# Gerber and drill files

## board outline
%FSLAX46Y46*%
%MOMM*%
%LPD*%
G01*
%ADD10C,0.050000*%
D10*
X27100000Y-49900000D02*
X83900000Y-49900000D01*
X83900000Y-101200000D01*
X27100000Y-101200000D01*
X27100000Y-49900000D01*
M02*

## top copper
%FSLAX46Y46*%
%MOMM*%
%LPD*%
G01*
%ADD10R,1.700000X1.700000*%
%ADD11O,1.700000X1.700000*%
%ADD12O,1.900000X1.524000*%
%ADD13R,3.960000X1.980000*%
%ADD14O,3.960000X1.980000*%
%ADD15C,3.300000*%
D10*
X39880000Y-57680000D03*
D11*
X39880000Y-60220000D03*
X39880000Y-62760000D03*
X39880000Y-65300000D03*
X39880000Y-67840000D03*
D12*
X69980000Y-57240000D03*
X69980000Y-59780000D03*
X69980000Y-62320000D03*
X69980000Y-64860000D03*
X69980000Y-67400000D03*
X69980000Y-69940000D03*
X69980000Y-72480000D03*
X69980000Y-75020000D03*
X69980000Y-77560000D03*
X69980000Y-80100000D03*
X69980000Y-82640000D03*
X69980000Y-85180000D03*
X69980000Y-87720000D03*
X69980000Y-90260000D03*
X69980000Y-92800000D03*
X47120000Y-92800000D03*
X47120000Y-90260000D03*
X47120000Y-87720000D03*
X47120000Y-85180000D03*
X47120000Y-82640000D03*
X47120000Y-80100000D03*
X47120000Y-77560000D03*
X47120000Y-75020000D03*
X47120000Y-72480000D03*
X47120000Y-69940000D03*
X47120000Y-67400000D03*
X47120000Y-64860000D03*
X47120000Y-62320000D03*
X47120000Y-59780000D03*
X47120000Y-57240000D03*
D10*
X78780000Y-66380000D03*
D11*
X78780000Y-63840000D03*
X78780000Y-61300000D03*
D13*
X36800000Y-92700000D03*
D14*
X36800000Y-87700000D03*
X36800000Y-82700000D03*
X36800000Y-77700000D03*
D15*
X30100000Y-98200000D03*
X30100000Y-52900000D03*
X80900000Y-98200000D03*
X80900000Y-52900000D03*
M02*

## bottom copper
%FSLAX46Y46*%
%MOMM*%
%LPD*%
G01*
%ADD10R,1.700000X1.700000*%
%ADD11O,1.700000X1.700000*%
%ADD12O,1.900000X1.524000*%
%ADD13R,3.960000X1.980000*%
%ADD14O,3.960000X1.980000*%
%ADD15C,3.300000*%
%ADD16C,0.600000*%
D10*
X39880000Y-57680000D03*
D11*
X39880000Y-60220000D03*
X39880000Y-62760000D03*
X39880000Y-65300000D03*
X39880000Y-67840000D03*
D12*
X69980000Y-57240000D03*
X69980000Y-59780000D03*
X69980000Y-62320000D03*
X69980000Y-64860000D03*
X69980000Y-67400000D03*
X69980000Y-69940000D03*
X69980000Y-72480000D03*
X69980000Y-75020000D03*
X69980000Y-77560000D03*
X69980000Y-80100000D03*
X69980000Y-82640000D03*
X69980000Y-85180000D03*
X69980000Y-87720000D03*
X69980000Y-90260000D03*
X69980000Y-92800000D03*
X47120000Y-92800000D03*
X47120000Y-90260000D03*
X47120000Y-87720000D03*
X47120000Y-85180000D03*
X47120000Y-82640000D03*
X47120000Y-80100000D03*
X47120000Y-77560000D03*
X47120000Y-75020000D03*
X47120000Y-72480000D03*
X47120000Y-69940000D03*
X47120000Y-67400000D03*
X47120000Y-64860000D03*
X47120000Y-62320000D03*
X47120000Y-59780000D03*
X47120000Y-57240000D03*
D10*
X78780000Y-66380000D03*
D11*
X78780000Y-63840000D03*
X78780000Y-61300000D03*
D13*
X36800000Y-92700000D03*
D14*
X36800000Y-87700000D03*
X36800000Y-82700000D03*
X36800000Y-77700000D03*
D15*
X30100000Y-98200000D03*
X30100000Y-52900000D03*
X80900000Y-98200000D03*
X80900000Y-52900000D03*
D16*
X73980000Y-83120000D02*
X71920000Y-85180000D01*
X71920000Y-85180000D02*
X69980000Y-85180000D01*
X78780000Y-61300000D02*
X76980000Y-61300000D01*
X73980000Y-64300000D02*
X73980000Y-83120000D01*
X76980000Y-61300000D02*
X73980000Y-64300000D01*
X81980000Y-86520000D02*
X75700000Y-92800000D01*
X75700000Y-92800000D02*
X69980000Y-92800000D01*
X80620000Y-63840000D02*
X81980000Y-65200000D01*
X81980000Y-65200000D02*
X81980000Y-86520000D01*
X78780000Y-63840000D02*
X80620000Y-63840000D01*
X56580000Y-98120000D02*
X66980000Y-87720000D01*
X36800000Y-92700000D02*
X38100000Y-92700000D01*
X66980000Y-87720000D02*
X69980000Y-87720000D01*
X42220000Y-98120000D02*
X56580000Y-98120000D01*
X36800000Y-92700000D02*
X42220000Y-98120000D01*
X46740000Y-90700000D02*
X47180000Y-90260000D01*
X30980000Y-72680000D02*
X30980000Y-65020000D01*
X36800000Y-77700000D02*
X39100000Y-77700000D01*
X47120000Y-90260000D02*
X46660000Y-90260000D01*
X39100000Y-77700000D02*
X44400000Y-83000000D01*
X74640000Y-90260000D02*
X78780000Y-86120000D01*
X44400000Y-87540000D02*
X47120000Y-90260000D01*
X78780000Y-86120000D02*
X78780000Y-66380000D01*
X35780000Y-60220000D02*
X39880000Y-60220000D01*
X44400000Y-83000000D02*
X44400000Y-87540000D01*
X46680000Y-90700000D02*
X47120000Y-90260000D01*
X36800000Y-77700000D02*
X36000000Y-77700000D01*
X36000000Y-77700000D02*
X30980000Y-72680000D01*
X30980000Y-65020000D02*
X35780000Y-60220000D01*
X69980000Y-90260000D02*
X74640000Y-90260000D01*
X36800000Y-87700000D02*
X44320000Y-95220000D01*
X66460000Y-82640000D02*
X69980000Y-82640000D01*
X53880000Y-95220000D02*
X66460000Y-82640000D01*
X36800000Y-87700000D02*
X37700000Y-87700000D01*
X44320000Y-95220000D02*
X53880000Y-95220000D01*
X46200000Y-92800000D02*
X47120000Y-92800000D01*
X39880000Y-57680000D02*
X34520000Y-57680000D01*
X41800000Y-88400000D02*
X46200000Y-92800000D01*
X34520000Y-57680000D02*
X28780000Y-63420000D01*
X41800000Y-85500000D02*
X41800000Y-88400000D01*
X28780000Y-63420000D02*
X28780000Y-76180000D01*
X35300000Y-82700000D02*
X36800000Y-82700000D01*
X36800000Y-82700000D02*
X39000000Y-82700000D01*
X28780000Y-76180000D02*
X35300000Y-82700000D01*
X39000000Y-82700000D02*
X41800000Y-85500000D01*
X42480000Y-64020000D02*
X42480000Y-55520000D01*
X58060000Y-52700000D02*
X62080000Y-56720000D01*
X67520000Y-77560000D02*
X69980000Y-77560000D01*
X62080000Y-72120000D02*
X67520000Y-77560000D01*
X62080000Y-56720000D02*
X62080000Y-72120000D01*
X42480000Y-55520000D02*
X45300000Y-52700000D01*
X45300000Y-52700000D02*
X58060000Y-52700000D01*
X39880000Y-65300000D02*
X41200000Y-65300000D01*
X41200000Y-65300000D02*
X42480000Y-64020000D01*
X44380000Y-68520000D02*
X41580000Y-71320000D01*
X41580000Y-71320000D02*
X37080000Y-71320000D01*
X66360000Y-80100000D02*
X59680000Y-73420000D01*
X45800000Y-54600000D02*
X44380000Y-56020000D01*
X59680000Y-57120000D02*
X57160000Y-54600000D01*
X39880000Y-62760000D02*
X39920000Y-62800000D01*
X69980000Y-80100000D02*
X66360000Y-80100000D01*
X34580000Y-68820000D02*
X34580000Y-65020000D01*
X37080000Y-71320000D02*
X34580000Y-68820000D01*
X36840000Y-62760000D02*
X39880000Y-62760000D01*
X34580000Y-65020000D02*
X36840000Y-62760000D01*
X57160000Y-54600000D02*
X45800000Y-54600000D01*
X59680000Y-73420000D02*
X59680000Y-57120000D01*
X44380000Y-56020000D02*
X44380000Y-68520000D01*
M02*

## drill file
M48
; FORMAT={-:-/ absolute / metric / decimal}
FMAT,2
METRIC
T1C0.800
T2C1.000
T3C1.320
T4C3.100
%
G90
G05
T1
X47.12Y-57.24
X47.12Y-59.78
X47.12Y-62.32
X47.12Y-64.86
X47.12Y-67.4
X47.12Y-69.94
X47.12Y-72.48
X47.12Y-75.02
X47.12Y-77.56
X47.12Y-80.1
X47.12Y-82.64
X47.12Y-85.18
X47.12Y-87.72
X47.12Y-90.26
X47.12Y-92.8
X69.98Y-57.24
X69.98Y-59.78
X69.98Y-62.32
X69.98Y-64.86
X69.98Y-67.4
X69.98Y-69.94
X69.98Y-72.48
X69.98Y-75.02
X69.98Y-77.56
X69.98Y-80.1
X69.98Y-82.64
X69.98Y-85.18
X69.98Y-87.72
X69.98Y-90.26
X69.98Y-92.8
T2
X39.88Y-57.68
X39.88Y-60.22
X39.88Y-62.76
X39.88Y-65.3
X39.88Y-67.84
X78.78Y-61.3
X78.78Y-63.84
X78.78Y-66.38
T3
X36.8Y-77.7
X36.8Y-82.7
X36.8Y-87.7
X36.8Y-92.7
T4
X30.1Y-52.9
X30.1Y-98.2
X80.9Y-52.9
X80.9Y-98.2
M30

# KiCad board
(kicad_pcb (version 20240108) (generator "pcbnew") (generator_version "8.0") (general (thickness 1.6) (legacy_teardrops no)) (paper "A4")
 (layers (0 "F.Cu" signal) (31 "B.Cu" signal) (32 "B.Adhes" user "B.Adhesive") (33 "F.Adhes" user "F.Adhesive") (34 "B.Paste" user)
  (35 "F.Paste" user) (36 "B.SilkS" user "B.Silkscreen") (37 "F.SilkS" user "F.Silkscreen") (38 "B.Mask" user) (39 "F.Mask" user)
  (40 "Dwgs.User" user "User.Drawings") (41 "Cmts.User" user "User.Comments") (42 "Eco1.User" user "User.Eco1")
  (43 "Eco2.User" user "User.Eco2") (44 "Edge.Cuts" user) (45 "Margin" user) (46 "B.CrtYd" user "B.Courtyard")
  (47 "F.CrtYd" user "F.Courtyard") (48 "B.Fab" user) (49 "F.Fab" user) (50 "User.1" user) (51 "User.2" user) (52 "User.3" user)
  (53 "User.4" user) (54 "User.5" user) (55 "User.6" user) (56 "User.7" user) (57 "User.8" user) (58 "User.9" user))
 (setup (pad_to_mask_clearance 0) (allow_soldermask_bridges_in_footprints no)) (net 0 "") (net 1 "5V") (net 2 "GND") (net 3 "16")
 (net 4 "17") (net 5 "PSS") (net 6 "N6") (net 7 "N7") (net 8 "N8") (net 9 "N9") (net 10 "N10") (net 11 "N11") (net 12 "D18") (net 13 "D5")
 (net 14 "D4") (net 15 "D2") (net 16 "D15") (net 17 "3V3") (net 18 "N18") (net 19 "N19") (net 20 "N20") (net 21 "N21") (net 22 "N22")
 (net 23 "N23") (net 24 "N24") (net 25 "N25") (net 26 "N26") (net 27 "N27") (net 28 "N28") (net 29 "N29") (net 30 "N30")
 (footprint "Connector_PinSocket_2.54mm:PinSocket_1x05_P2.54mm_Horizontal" (layer "F.Cu") (at 39.88 57.68)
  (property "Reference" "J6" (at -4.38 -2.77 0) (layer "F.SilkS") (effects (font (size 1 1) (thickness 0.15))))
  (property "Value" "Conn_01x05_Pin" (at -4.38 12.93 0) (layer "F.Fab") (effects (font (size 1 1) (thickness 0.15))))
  (pad "1" thru_hole rect (at 0 0) (size 1.7 1.7) (drill 1) (layers "*.Cu" "*.Mask") (remove_unused_layers no) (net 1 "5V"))
  (pad "2" thru_hole oval (at 0 2.54) (size 1.7 1.7) (drill 1) (layers "*.Cu" "*.Mask") (remove_unused_layers no) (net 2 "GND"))
  (pad "3" thru_hole oval (at 0 5.08) (size 1.7 1.7) (drill 1) (layers "*.Cu" "*.Mask") (remove_unused_layers no) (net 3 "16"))
  (pad "4" thru_hole oval (at 0 7.62) (size 1.7 1.7) (drill 1) (layers "*.Cu" "*.Mask") (remove_unused_layers no) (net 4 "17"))
  (pad "5" thru_hole oval (at 0 10.16) (size 1.7 1.7) (drill 1) (layers "*.Cu" "*.Mask") (remove_unused_layers no) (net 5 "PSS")))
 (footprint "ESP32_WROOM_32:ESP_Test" (layer "F.Cu") (at 58.68 74.64 -90)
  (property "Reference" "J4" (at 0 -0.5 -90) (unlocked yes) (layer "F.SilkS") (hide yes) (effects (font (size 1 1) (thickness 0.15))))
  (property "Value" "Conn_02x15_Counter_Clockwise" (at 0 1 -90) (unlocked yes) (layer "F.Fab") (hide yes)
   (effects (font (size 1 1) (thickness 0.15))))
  (pad "1" thru_hole oval (at -17.4 -11.3 270) (size 1.524 1.9) (drill 0.8) (layers "*.Cu" "*.Mask") (remove_unused_layers no) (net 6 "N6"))
  (pad "2" thru_hole oval (at -14.86 -11.3 270) (size 1.524 1.9) (drill 0.8) (layers "*.Cu" "*.Mask") (remove_unused_layers no) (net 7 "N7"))
  (pad "3" thru_hole oval (at -12.32 -11.3 270) (size 1.524 1.9) (drill 0.8) (layers "*.Cu" "*.Mask") (remove_unused_layers no) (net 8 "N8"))
  (pad "4" thru_hole oval (at -9.78 -11.3 270) (size 1.524 1.9) (drill 0.8) (layers "*.Cu" "*.Mask") (remove_unused_layers no) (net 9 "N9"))
  (pad "5" thru_hole oval (at -7.24 -11.3 270) (size 1.524 1.9) (drill 0.8) (layers "*.Cu" "*.Mask") (remove_unused_layers no)
   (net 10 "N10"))
  (pad "6" thru_hole oval (at -4.7 -11.3 270) (size 1.524 1.9) (drill 0.8) (layers "*.Cu" "*.Mask") (remove_unused_layers no) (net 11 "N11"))
  (pad "7" thru_hole oval (at -2.16 -11.3 270) (size 1.524 1.9) (drill 0.8) (layers "*.Cu" "*.Mask") (remove_unused_layers no)
   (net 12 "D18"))
  (pad "8" thru_hole oval (at 0.38 -11.3 270) (size 1.524 1.9) (drill 0.8) (layers "*.Cu" "*.Mask") (remove_unused_layers no) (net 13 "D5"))
  (pad "9" thru_hole oval (at 2.92 -11.3 270) (size 1.524 1.9) (drill 0.8) (layers "*.Cu" "*.Mask") (remove_unused_layers no) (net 4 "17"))
  (pad "10" thru_hole oval (at 5.46 -11.3 270) (size 1.524 1.9) (drill 0.8) (layers "*.Cu" "*.Mask") (remove_unused_layers no) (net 3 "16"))
  (pad "11" thru_hole oval (at 8 -11.3 270) (size 1.524 1.9) (drill 0.8) (layers "*.Cu" "*.Mask") (remove_unused_layers no) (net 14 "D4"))
  (pad "12" thru_hole oval (at 10.54 -11.3 270) (size 1.524 1.9) (drill 0.8) (layers "*.Cu" "*.Mask") (remove_unused_layers no)
   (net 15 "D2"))
  (pad "13" thru_hole oval (at 13.08 -11.3 270) (size 1.524 1.9) (drill 0.8) (layers "*.Cu" "*.Mask") (remove_unused_layers no)
   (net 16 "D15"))
  (pad "14" thru_hole oval (at 15.62 -11.3 270) (size 1.524 1.9) (drill 0.8) (layers "*.Cu" "*.Mask") (remove_unused_layers no)
   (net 2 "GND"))
  (pad "15" thru_hole oval (at 18.16 -11.3 270) (size 1.524 1.9) (drill 0.8) (layers "*.Cu" "*.Mask") (remove_unused_layers no)
   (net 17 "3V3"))
  (pad "16" thru_hole oval (at 18.16 11.56 270) (size 1.524 1.9) (drill 0.8) (layers "*.Cu" "*.Mask") (remove_unused_layers no) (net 1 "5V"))
  (pad "17" thru_hole oval (at 15.62 11.56 270) (size 1.524 1.9) (drill 0.8) (layers "*.Cu" "*.Mask") (remove_unused_layers no)
   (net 2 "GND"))
  (pad "18" thru_hole oval (at 13.08 11.56 270) (size 1.524 1.9) (drill 0.8) (layers "*.Cu" "*.Mask") (remove_unused_layers no)
   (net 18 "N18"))
  (pad "19" thru_hole oval (at 10.54 11.56 270) (size 1.524 1.9) (drill 0.8) (layers "*.Cu" "*.Mask") (remove_unused_layers no)
   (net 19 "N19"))
  (pad "20" thru_hole oval (at 8 11.56 270) (size 1.524 1.9) (drill 0.8) (layers "*.Cu" "*.Mask") (remove_unused_layers no) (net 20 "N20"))
  (pad "21" thru_hole oval (at 5.46 11.56 270) (size 1.524 1.9) (drill 0.8) (layers "*.Cu" "*.Mask") (remove_unused_layers no)
   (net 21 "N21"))
  (pad "22" thru_hole oval (at 2.92 11.56 270) (size 1.524 1.9) (drill 0.8) (layers "*.Cu" "*.Mask") (remove_unused_layers no)
   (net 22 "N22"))
  (pad "23" thru_hole oval (at 0.38 11.56 270) (size 1.524 1.9) (drill 0.8) (layers "*.Cu" "*.Mask") (remove_unused_layers no)
   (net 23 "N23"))
  (pad "24" thru_hole oval (at -2.16 11.56 270) (size 1.524 1.9) (drill 0.8) (layers "*.Cu" "*.Mask") (remove_unused_layers no)
   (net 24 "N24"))
  (pad "25" thru_hole oval (at -4.7 11.56 270) (size 1.524 1.9) (drill 0.8) (layers "*.Cu" "*.Mask") (remove_unused_layers no)
   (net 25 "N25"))
  (pad "26" thru_hole oval (at -7.24 11.56 270) (size 1.524 1.9) (drill 0.8) (layers "*.Cu" "*.Mask") (remove_unused_layers no)
   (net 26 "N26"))
  (pad "27" thru_hole oval (at -9.78 11.56 270) (size 1.524 1.9) (drill 0.8) (layers "*.Cu" "*.Mask") (remove_unused_layers no)
   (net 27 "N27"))
  (pad "28" thru_hole oval (at -12.32 11.56 270) (size 1.524 1.9) (drill 0.8) (layers "*.Cu" "*.Mask") (remove_unused_layers no)
   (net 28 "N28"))
  (pad "29" thru_hole oval (at -14.86 11.56 270) (size 1.524 1.9) (drill 0.8) (layers "*.Cu" "*.Mask") (remove_unused_layers no)
   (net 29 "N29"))
  (pad "30" thru_hole oval (at -17.4 11.56 270) (size 1.524 1.9) (drill 0.8) (layers "*.Cu" "*.Mask") (remove_unused_layers no)
   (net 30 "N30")))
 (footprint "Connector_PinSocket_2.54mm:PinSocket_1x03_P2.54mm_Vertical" (layer "F.Cu") (at 78.78 66.38 180)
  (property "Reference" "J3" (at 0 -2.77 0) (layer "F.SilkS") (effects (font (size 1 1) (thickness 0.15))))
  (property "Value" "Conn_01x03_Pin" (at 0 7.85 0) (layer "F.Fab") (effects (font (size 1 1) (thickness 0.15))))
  (pad "1" thru_hole rect (at 0 0 180) (size 1.7 1.7) (drill 1) (layers "*.Cu" "*.Mask") (remove_unused_layers no) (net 2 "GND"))
  (pad "2" thru_hole oval (at 0 2.54 180) (size 1.7 1.7) (drill 1) (layers "*.Cu" "*.Mask") (remove_unused_layers no) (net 17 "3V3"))
  (pad "3" thru_hole oval (at 0 5.08 180) (size 1.7 1.7) (drill 1) (layers "*.Cu" "*.Mask") (remove_unused_layers no) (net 15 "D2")))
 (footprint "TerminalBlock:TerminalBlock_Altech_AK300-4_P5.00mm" (layer "F.Cu") (at 36.8 92.7 90)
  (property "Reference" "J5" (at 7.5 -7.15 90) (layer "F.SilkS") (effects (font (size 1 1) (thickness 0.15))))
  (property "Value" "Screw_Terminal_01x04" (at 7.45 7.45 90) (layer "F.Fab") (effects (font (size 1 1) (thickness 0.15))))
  (pad "1" thru_hole rect (at 0 0 90) (size 1.98 3.96) (drill 1.32) (layers "*.Cu" "*.Mask") (remove_unused_layers no) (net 16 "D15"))
  (pad "2" thru_hole oval (at 5 0 90) (size 1.98 3.96) (drill 1.32) (layers "*.Cu" "*.Mask") (remove_unused_layers no) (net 14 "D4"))
  (pad "3" thru_hole oval (at 10 0 90) (size 1.98 3.96) (drill 1.32) (layers "*.Cu" "*.Mask") (remove_unused_layers no) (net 1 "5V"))
  (pad "4" thru_hole oval (at 15 0 90) (size 1.98 3.96) (drill 1.32) (layers "*.Cu" "*.Mask") (remove_unused_layers no) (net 2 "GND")))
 (gr_rect (start 27.1 49.9) (end 83.9 101.2) (stroke (width 0.05) (type default)) (fill none) (layer "Edge.Cuts"))
 (via (at 30.1 98.2) (size 3.3) (drill 3.1) (layers "F.Cu" "B.Cu") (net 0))
 (via (at 30.1 52.9) (size 3.3) (drill 3.1) (layers "F.Cu" "B.Cu") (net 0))
 (via (at 80.9 98.2) (size 3.3) (drill 3.1) (layers "F.Cu" "B.Cu") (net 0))
 (via (at 80.9 52.9) (size 3.3) (drill 3.1) (layers "F.Cu" "B.Cu") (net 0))
 (segment (start 73.98 83.12) (end 71.92 85.18) (width 0.6) (layer "B.Cu") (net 15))
 (segment (start 71.92 85.18) (end 69.98 85.18) (width 0.6) (layer "B.Cu") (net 15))
 (segment (start 78.78 61.3) (end 76.98 61.3) (width 0.6) (layer "B.Cu") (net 15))
 (segment (start 73.98 64.3) (end 73.98 83.12) (width 0.6) (layer "B.Cu") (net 15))
 (segment (start 76.98 61.3) (end 73.98 64.3) (width 0.6) (layer "B.Cu") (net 15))
 (segment (start 81.98 86.52) (end 75.7 92.8) (width 0.6) (layer "B.Cu") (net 17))
 (segment (start 75.7 92.8) (end 69.98 92.8) (width 0.6) (layer "B.Cu") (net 17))
 (segment (start 80.62 63.84) (end 81.98 65.2) (width 0.6) (layer "B.Cu") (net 17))
 (segment (start 81.98 65.2) (end 81.98 86.52) (width 0.6) (layer "B.Cu") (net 17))
 (segment (start 78.78 63.84) (end 80.62 63.84) (width 0.6) (layer "B.Cu") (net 17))
 (segment (start 56.58 98.12) (end 66.98 87.72) (width 0.6) (layer "B.Cu") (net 16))
 (segment (start 36.8 92.7) (end 38.1 92.7) (width 0.6) (layer "B.Cu") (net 16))
 (segment (start 66.98 87.72) (end 69.98 87.72) (width 0.6) (layer "B.Cu") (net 16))
 (segment (start 42.22 98.12) (end 56.58 98.12) (width 0.6) (layer "B.Cu") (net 16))
 (segment (start 36.8 92.7) (end 42.22 98.12) (width 0.6) (layer "B.Cu") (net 16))
 (segment (start 46.74 90.7) (end 47.18 90.26) (width 0.6) (layer "B.Cu") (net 2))
 (segment (start 30.98 72.68) (end 30.98 65.02) (width 0.6) (layer "B.Cu") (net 2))
 (segment (start 36.8 77.7) (end 39.1 77.7) (width 0.6) (layer "B.Cu") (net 2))
 (segment (start 47.12 90.26) (end 46.66 90.26) (width 0.6) (layer "B.Cu") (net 2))
 (segment (start 39.1 77.7) (end 44.4 83) (width 0.6) (layer "B.Cu") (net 2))
 (segment (start 74.64 90.26) (end 78.78 86.12) (width 0.6) (layer "B.Cu") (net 2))
 (segment (start 44.4 87.54) (end 47.12 90.26) (width 0.6) (layer "B.Cu") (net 2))
 (segment (start 78.78 86.12) (end 78.78 66.38) (width 0.6) (layer "B.Cu") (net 2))
 (segment (start 35.78 60.22) (end 39.88 60.22) (width 0.6) (layer "B.Cu") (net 2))
 (segment (start 44.4 83) (end 44.4 87.54) (width 0.6) (layer "B.Cu") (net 2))
 (segment (start 46.68 90.7) (end 47.12 90.26) (width 0.6) (layer "B.Cu") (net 2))
 (segment (start 36.8 77.7) (end 36 77.7) (width 0.6) (layer "B.Cu") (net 2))
 (segment (start 36 77.7) (end 30.98 72.68) (width 0.6) (layer "B.Cu") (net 2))
 (segment (start 30.98 65.02) (end 35.78 60.22) (width 0.6) (layer "B.Cu") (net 2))
 (segment (start 69.98 90.26) (end 74.64 90.26) (width 0.6) (layer "B.Cu") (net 2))
 (segment (start 36.8 87.7) (end 44.32 95.22) (width 0.6) (layer "B.Cu") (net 14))
 (segment (start 66.46 82.64) (end 69.98 82.64) (width 0.6) (layer "B.Cu") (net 14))
 (segment (start 53.88 95.22) (end 66.46 82.64) (width 0.6) (layer "B.Cu") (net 14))
 (segment (start 36.8 87.7) (end 37.7 87.7) (width 0.6) (layer "B.Cu") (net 14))
 (segment (start 44.32 95.22) (end 53.88 95.22) (width 0.6) (layer "B.Cu") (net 14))
 (segment (start 46.2 92.8) (end 47.12 92.8) (width 0.6) (layer "B.Cu") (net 1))
 (segment (start 39.88 57.68) (end 34.52 57.68) (width 0.6) (layer "B.Cu") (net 1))
 (segment (start 41.8 88.4) (end 46.2 92.8) (width 0.6) (layer "B.Cu") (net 1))
 (segment (start 34.52 57.68) (end 28.78 63.42) (width 0.6) (layer "B.Cu") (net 1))
 (segment (start 41.8 85.5) (end 41.8 88.4) (width 0.6) (layer "B.Cu") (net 1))
 (segment (start 28.78 63.42) (end 28.78 76.18) (width 0.6) (layer "B.Cu") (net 1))
 (segment (start 35.3 82.7) (end 36.8 82.7) (width 0.6) (layer "B.Cu") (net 1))
 (segment (start 36.8 82.7) (end 39 82.7) (width 0.6) (layer "B.Cu") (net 1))
 (segment (start 28.78 76.18) (end 35.3 82.7) (width 0.6) (layer "B.Cu") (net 1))
 (segment (start 39 82.7) (end 41.8 85.5) (width 0.6) (layer "B.Cu") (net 1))
 (segment (start 42.48 64.02) (end 42.48 55.52) (width 0.6) (layer "B.Cu") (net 4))
 (segment (start 58.06 52.7) (end 62.08 56.72) (width 0.6) (layer "B.Cu") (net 4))
 (segment (start 67.52 77.56) (end 69.98 77.56) (width 0.6) (layer "B.Cu") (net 4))
 (segment (start 62.08 72.12) (end 67.52 77.56) (width 0.6) (layer "B.Cu") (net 4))
 (segment (start 62.08 56.72) (end 62.08 72.12) (width 0.6) (layer "B.Cu") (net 4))
 (segment (start 42.48 55.52) (end 45.3 52.7) (width 0.6) (layer "B.Cu") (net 4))
 (segment (start 45.3 52.7) (end 58.06 52.7) (width 0.6) (layer "B.Cu") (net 4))
 (segment (start 39.88 65.3) (end 41.2 65.3) (width 0.6) (layer "B.Cu") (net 4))
 (segment (start 41.2 65.3) (end 42.48 64.02) (width 0.6) (layer "B.Cu") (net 4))
 (segment (start 44.38 68.52) (end 41.58 71.32) (width 0.6) (layer "B.Cu") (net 3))
 (segment (start 41.58 71.32) (end 37.08 71.32) (width 0.6) (layer "B.Cu") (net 3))
 (segment (start 66.36 80.1) (end 59.68 73.42) (width 0.6) (layer "B.Cu") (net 3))
 (segment (start 45.8 54.6) (end 44.38 56.02) (width 0.6) (layer "B.Cu") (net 3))
 (segment (start 59.68 57.12) (end 57.16 54.6) (width 0.6) (layer "B.Cu") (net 3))
 (segment (start 39.88 62.76) (end 39.92 62.8) (width 0.6) (layer "B.Cu") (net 3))
 (segment (start 69.98 80.1) (end 66.36 80.1) (width 0.6) (layer "B.Cu") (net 3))
 (segment (start 34.58 68.82) (end 34.58 65.02) (width 0.6) (layer "B.Cu") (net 3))
 (segment (start 37.08 71.32) (end 34.58 68.82) (width 0.6) (layer "B.Cu") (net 3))
 (segment (start 36.84 62.76) (end 39.88 62.76) (width 0.6) (layer "B.Cu") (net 3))
 (segment (start 34.58 65.02) (end 36.84 62.76) (width 0.6) (layer "B.Cu") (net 3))
 (segment (start 57.16 54.6) (end 45.8 54.6) (width 0.6) (layer "B.Cu") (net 3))
 (segment (start 59.68 73.42) (end 59.68 57.12) (width 0.6) (layer "B.Cu") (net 3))
 (segment (start 44.38 56.02) (end 44.38 68.52) (width 0.6) (layer "B.Cu") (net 3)))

